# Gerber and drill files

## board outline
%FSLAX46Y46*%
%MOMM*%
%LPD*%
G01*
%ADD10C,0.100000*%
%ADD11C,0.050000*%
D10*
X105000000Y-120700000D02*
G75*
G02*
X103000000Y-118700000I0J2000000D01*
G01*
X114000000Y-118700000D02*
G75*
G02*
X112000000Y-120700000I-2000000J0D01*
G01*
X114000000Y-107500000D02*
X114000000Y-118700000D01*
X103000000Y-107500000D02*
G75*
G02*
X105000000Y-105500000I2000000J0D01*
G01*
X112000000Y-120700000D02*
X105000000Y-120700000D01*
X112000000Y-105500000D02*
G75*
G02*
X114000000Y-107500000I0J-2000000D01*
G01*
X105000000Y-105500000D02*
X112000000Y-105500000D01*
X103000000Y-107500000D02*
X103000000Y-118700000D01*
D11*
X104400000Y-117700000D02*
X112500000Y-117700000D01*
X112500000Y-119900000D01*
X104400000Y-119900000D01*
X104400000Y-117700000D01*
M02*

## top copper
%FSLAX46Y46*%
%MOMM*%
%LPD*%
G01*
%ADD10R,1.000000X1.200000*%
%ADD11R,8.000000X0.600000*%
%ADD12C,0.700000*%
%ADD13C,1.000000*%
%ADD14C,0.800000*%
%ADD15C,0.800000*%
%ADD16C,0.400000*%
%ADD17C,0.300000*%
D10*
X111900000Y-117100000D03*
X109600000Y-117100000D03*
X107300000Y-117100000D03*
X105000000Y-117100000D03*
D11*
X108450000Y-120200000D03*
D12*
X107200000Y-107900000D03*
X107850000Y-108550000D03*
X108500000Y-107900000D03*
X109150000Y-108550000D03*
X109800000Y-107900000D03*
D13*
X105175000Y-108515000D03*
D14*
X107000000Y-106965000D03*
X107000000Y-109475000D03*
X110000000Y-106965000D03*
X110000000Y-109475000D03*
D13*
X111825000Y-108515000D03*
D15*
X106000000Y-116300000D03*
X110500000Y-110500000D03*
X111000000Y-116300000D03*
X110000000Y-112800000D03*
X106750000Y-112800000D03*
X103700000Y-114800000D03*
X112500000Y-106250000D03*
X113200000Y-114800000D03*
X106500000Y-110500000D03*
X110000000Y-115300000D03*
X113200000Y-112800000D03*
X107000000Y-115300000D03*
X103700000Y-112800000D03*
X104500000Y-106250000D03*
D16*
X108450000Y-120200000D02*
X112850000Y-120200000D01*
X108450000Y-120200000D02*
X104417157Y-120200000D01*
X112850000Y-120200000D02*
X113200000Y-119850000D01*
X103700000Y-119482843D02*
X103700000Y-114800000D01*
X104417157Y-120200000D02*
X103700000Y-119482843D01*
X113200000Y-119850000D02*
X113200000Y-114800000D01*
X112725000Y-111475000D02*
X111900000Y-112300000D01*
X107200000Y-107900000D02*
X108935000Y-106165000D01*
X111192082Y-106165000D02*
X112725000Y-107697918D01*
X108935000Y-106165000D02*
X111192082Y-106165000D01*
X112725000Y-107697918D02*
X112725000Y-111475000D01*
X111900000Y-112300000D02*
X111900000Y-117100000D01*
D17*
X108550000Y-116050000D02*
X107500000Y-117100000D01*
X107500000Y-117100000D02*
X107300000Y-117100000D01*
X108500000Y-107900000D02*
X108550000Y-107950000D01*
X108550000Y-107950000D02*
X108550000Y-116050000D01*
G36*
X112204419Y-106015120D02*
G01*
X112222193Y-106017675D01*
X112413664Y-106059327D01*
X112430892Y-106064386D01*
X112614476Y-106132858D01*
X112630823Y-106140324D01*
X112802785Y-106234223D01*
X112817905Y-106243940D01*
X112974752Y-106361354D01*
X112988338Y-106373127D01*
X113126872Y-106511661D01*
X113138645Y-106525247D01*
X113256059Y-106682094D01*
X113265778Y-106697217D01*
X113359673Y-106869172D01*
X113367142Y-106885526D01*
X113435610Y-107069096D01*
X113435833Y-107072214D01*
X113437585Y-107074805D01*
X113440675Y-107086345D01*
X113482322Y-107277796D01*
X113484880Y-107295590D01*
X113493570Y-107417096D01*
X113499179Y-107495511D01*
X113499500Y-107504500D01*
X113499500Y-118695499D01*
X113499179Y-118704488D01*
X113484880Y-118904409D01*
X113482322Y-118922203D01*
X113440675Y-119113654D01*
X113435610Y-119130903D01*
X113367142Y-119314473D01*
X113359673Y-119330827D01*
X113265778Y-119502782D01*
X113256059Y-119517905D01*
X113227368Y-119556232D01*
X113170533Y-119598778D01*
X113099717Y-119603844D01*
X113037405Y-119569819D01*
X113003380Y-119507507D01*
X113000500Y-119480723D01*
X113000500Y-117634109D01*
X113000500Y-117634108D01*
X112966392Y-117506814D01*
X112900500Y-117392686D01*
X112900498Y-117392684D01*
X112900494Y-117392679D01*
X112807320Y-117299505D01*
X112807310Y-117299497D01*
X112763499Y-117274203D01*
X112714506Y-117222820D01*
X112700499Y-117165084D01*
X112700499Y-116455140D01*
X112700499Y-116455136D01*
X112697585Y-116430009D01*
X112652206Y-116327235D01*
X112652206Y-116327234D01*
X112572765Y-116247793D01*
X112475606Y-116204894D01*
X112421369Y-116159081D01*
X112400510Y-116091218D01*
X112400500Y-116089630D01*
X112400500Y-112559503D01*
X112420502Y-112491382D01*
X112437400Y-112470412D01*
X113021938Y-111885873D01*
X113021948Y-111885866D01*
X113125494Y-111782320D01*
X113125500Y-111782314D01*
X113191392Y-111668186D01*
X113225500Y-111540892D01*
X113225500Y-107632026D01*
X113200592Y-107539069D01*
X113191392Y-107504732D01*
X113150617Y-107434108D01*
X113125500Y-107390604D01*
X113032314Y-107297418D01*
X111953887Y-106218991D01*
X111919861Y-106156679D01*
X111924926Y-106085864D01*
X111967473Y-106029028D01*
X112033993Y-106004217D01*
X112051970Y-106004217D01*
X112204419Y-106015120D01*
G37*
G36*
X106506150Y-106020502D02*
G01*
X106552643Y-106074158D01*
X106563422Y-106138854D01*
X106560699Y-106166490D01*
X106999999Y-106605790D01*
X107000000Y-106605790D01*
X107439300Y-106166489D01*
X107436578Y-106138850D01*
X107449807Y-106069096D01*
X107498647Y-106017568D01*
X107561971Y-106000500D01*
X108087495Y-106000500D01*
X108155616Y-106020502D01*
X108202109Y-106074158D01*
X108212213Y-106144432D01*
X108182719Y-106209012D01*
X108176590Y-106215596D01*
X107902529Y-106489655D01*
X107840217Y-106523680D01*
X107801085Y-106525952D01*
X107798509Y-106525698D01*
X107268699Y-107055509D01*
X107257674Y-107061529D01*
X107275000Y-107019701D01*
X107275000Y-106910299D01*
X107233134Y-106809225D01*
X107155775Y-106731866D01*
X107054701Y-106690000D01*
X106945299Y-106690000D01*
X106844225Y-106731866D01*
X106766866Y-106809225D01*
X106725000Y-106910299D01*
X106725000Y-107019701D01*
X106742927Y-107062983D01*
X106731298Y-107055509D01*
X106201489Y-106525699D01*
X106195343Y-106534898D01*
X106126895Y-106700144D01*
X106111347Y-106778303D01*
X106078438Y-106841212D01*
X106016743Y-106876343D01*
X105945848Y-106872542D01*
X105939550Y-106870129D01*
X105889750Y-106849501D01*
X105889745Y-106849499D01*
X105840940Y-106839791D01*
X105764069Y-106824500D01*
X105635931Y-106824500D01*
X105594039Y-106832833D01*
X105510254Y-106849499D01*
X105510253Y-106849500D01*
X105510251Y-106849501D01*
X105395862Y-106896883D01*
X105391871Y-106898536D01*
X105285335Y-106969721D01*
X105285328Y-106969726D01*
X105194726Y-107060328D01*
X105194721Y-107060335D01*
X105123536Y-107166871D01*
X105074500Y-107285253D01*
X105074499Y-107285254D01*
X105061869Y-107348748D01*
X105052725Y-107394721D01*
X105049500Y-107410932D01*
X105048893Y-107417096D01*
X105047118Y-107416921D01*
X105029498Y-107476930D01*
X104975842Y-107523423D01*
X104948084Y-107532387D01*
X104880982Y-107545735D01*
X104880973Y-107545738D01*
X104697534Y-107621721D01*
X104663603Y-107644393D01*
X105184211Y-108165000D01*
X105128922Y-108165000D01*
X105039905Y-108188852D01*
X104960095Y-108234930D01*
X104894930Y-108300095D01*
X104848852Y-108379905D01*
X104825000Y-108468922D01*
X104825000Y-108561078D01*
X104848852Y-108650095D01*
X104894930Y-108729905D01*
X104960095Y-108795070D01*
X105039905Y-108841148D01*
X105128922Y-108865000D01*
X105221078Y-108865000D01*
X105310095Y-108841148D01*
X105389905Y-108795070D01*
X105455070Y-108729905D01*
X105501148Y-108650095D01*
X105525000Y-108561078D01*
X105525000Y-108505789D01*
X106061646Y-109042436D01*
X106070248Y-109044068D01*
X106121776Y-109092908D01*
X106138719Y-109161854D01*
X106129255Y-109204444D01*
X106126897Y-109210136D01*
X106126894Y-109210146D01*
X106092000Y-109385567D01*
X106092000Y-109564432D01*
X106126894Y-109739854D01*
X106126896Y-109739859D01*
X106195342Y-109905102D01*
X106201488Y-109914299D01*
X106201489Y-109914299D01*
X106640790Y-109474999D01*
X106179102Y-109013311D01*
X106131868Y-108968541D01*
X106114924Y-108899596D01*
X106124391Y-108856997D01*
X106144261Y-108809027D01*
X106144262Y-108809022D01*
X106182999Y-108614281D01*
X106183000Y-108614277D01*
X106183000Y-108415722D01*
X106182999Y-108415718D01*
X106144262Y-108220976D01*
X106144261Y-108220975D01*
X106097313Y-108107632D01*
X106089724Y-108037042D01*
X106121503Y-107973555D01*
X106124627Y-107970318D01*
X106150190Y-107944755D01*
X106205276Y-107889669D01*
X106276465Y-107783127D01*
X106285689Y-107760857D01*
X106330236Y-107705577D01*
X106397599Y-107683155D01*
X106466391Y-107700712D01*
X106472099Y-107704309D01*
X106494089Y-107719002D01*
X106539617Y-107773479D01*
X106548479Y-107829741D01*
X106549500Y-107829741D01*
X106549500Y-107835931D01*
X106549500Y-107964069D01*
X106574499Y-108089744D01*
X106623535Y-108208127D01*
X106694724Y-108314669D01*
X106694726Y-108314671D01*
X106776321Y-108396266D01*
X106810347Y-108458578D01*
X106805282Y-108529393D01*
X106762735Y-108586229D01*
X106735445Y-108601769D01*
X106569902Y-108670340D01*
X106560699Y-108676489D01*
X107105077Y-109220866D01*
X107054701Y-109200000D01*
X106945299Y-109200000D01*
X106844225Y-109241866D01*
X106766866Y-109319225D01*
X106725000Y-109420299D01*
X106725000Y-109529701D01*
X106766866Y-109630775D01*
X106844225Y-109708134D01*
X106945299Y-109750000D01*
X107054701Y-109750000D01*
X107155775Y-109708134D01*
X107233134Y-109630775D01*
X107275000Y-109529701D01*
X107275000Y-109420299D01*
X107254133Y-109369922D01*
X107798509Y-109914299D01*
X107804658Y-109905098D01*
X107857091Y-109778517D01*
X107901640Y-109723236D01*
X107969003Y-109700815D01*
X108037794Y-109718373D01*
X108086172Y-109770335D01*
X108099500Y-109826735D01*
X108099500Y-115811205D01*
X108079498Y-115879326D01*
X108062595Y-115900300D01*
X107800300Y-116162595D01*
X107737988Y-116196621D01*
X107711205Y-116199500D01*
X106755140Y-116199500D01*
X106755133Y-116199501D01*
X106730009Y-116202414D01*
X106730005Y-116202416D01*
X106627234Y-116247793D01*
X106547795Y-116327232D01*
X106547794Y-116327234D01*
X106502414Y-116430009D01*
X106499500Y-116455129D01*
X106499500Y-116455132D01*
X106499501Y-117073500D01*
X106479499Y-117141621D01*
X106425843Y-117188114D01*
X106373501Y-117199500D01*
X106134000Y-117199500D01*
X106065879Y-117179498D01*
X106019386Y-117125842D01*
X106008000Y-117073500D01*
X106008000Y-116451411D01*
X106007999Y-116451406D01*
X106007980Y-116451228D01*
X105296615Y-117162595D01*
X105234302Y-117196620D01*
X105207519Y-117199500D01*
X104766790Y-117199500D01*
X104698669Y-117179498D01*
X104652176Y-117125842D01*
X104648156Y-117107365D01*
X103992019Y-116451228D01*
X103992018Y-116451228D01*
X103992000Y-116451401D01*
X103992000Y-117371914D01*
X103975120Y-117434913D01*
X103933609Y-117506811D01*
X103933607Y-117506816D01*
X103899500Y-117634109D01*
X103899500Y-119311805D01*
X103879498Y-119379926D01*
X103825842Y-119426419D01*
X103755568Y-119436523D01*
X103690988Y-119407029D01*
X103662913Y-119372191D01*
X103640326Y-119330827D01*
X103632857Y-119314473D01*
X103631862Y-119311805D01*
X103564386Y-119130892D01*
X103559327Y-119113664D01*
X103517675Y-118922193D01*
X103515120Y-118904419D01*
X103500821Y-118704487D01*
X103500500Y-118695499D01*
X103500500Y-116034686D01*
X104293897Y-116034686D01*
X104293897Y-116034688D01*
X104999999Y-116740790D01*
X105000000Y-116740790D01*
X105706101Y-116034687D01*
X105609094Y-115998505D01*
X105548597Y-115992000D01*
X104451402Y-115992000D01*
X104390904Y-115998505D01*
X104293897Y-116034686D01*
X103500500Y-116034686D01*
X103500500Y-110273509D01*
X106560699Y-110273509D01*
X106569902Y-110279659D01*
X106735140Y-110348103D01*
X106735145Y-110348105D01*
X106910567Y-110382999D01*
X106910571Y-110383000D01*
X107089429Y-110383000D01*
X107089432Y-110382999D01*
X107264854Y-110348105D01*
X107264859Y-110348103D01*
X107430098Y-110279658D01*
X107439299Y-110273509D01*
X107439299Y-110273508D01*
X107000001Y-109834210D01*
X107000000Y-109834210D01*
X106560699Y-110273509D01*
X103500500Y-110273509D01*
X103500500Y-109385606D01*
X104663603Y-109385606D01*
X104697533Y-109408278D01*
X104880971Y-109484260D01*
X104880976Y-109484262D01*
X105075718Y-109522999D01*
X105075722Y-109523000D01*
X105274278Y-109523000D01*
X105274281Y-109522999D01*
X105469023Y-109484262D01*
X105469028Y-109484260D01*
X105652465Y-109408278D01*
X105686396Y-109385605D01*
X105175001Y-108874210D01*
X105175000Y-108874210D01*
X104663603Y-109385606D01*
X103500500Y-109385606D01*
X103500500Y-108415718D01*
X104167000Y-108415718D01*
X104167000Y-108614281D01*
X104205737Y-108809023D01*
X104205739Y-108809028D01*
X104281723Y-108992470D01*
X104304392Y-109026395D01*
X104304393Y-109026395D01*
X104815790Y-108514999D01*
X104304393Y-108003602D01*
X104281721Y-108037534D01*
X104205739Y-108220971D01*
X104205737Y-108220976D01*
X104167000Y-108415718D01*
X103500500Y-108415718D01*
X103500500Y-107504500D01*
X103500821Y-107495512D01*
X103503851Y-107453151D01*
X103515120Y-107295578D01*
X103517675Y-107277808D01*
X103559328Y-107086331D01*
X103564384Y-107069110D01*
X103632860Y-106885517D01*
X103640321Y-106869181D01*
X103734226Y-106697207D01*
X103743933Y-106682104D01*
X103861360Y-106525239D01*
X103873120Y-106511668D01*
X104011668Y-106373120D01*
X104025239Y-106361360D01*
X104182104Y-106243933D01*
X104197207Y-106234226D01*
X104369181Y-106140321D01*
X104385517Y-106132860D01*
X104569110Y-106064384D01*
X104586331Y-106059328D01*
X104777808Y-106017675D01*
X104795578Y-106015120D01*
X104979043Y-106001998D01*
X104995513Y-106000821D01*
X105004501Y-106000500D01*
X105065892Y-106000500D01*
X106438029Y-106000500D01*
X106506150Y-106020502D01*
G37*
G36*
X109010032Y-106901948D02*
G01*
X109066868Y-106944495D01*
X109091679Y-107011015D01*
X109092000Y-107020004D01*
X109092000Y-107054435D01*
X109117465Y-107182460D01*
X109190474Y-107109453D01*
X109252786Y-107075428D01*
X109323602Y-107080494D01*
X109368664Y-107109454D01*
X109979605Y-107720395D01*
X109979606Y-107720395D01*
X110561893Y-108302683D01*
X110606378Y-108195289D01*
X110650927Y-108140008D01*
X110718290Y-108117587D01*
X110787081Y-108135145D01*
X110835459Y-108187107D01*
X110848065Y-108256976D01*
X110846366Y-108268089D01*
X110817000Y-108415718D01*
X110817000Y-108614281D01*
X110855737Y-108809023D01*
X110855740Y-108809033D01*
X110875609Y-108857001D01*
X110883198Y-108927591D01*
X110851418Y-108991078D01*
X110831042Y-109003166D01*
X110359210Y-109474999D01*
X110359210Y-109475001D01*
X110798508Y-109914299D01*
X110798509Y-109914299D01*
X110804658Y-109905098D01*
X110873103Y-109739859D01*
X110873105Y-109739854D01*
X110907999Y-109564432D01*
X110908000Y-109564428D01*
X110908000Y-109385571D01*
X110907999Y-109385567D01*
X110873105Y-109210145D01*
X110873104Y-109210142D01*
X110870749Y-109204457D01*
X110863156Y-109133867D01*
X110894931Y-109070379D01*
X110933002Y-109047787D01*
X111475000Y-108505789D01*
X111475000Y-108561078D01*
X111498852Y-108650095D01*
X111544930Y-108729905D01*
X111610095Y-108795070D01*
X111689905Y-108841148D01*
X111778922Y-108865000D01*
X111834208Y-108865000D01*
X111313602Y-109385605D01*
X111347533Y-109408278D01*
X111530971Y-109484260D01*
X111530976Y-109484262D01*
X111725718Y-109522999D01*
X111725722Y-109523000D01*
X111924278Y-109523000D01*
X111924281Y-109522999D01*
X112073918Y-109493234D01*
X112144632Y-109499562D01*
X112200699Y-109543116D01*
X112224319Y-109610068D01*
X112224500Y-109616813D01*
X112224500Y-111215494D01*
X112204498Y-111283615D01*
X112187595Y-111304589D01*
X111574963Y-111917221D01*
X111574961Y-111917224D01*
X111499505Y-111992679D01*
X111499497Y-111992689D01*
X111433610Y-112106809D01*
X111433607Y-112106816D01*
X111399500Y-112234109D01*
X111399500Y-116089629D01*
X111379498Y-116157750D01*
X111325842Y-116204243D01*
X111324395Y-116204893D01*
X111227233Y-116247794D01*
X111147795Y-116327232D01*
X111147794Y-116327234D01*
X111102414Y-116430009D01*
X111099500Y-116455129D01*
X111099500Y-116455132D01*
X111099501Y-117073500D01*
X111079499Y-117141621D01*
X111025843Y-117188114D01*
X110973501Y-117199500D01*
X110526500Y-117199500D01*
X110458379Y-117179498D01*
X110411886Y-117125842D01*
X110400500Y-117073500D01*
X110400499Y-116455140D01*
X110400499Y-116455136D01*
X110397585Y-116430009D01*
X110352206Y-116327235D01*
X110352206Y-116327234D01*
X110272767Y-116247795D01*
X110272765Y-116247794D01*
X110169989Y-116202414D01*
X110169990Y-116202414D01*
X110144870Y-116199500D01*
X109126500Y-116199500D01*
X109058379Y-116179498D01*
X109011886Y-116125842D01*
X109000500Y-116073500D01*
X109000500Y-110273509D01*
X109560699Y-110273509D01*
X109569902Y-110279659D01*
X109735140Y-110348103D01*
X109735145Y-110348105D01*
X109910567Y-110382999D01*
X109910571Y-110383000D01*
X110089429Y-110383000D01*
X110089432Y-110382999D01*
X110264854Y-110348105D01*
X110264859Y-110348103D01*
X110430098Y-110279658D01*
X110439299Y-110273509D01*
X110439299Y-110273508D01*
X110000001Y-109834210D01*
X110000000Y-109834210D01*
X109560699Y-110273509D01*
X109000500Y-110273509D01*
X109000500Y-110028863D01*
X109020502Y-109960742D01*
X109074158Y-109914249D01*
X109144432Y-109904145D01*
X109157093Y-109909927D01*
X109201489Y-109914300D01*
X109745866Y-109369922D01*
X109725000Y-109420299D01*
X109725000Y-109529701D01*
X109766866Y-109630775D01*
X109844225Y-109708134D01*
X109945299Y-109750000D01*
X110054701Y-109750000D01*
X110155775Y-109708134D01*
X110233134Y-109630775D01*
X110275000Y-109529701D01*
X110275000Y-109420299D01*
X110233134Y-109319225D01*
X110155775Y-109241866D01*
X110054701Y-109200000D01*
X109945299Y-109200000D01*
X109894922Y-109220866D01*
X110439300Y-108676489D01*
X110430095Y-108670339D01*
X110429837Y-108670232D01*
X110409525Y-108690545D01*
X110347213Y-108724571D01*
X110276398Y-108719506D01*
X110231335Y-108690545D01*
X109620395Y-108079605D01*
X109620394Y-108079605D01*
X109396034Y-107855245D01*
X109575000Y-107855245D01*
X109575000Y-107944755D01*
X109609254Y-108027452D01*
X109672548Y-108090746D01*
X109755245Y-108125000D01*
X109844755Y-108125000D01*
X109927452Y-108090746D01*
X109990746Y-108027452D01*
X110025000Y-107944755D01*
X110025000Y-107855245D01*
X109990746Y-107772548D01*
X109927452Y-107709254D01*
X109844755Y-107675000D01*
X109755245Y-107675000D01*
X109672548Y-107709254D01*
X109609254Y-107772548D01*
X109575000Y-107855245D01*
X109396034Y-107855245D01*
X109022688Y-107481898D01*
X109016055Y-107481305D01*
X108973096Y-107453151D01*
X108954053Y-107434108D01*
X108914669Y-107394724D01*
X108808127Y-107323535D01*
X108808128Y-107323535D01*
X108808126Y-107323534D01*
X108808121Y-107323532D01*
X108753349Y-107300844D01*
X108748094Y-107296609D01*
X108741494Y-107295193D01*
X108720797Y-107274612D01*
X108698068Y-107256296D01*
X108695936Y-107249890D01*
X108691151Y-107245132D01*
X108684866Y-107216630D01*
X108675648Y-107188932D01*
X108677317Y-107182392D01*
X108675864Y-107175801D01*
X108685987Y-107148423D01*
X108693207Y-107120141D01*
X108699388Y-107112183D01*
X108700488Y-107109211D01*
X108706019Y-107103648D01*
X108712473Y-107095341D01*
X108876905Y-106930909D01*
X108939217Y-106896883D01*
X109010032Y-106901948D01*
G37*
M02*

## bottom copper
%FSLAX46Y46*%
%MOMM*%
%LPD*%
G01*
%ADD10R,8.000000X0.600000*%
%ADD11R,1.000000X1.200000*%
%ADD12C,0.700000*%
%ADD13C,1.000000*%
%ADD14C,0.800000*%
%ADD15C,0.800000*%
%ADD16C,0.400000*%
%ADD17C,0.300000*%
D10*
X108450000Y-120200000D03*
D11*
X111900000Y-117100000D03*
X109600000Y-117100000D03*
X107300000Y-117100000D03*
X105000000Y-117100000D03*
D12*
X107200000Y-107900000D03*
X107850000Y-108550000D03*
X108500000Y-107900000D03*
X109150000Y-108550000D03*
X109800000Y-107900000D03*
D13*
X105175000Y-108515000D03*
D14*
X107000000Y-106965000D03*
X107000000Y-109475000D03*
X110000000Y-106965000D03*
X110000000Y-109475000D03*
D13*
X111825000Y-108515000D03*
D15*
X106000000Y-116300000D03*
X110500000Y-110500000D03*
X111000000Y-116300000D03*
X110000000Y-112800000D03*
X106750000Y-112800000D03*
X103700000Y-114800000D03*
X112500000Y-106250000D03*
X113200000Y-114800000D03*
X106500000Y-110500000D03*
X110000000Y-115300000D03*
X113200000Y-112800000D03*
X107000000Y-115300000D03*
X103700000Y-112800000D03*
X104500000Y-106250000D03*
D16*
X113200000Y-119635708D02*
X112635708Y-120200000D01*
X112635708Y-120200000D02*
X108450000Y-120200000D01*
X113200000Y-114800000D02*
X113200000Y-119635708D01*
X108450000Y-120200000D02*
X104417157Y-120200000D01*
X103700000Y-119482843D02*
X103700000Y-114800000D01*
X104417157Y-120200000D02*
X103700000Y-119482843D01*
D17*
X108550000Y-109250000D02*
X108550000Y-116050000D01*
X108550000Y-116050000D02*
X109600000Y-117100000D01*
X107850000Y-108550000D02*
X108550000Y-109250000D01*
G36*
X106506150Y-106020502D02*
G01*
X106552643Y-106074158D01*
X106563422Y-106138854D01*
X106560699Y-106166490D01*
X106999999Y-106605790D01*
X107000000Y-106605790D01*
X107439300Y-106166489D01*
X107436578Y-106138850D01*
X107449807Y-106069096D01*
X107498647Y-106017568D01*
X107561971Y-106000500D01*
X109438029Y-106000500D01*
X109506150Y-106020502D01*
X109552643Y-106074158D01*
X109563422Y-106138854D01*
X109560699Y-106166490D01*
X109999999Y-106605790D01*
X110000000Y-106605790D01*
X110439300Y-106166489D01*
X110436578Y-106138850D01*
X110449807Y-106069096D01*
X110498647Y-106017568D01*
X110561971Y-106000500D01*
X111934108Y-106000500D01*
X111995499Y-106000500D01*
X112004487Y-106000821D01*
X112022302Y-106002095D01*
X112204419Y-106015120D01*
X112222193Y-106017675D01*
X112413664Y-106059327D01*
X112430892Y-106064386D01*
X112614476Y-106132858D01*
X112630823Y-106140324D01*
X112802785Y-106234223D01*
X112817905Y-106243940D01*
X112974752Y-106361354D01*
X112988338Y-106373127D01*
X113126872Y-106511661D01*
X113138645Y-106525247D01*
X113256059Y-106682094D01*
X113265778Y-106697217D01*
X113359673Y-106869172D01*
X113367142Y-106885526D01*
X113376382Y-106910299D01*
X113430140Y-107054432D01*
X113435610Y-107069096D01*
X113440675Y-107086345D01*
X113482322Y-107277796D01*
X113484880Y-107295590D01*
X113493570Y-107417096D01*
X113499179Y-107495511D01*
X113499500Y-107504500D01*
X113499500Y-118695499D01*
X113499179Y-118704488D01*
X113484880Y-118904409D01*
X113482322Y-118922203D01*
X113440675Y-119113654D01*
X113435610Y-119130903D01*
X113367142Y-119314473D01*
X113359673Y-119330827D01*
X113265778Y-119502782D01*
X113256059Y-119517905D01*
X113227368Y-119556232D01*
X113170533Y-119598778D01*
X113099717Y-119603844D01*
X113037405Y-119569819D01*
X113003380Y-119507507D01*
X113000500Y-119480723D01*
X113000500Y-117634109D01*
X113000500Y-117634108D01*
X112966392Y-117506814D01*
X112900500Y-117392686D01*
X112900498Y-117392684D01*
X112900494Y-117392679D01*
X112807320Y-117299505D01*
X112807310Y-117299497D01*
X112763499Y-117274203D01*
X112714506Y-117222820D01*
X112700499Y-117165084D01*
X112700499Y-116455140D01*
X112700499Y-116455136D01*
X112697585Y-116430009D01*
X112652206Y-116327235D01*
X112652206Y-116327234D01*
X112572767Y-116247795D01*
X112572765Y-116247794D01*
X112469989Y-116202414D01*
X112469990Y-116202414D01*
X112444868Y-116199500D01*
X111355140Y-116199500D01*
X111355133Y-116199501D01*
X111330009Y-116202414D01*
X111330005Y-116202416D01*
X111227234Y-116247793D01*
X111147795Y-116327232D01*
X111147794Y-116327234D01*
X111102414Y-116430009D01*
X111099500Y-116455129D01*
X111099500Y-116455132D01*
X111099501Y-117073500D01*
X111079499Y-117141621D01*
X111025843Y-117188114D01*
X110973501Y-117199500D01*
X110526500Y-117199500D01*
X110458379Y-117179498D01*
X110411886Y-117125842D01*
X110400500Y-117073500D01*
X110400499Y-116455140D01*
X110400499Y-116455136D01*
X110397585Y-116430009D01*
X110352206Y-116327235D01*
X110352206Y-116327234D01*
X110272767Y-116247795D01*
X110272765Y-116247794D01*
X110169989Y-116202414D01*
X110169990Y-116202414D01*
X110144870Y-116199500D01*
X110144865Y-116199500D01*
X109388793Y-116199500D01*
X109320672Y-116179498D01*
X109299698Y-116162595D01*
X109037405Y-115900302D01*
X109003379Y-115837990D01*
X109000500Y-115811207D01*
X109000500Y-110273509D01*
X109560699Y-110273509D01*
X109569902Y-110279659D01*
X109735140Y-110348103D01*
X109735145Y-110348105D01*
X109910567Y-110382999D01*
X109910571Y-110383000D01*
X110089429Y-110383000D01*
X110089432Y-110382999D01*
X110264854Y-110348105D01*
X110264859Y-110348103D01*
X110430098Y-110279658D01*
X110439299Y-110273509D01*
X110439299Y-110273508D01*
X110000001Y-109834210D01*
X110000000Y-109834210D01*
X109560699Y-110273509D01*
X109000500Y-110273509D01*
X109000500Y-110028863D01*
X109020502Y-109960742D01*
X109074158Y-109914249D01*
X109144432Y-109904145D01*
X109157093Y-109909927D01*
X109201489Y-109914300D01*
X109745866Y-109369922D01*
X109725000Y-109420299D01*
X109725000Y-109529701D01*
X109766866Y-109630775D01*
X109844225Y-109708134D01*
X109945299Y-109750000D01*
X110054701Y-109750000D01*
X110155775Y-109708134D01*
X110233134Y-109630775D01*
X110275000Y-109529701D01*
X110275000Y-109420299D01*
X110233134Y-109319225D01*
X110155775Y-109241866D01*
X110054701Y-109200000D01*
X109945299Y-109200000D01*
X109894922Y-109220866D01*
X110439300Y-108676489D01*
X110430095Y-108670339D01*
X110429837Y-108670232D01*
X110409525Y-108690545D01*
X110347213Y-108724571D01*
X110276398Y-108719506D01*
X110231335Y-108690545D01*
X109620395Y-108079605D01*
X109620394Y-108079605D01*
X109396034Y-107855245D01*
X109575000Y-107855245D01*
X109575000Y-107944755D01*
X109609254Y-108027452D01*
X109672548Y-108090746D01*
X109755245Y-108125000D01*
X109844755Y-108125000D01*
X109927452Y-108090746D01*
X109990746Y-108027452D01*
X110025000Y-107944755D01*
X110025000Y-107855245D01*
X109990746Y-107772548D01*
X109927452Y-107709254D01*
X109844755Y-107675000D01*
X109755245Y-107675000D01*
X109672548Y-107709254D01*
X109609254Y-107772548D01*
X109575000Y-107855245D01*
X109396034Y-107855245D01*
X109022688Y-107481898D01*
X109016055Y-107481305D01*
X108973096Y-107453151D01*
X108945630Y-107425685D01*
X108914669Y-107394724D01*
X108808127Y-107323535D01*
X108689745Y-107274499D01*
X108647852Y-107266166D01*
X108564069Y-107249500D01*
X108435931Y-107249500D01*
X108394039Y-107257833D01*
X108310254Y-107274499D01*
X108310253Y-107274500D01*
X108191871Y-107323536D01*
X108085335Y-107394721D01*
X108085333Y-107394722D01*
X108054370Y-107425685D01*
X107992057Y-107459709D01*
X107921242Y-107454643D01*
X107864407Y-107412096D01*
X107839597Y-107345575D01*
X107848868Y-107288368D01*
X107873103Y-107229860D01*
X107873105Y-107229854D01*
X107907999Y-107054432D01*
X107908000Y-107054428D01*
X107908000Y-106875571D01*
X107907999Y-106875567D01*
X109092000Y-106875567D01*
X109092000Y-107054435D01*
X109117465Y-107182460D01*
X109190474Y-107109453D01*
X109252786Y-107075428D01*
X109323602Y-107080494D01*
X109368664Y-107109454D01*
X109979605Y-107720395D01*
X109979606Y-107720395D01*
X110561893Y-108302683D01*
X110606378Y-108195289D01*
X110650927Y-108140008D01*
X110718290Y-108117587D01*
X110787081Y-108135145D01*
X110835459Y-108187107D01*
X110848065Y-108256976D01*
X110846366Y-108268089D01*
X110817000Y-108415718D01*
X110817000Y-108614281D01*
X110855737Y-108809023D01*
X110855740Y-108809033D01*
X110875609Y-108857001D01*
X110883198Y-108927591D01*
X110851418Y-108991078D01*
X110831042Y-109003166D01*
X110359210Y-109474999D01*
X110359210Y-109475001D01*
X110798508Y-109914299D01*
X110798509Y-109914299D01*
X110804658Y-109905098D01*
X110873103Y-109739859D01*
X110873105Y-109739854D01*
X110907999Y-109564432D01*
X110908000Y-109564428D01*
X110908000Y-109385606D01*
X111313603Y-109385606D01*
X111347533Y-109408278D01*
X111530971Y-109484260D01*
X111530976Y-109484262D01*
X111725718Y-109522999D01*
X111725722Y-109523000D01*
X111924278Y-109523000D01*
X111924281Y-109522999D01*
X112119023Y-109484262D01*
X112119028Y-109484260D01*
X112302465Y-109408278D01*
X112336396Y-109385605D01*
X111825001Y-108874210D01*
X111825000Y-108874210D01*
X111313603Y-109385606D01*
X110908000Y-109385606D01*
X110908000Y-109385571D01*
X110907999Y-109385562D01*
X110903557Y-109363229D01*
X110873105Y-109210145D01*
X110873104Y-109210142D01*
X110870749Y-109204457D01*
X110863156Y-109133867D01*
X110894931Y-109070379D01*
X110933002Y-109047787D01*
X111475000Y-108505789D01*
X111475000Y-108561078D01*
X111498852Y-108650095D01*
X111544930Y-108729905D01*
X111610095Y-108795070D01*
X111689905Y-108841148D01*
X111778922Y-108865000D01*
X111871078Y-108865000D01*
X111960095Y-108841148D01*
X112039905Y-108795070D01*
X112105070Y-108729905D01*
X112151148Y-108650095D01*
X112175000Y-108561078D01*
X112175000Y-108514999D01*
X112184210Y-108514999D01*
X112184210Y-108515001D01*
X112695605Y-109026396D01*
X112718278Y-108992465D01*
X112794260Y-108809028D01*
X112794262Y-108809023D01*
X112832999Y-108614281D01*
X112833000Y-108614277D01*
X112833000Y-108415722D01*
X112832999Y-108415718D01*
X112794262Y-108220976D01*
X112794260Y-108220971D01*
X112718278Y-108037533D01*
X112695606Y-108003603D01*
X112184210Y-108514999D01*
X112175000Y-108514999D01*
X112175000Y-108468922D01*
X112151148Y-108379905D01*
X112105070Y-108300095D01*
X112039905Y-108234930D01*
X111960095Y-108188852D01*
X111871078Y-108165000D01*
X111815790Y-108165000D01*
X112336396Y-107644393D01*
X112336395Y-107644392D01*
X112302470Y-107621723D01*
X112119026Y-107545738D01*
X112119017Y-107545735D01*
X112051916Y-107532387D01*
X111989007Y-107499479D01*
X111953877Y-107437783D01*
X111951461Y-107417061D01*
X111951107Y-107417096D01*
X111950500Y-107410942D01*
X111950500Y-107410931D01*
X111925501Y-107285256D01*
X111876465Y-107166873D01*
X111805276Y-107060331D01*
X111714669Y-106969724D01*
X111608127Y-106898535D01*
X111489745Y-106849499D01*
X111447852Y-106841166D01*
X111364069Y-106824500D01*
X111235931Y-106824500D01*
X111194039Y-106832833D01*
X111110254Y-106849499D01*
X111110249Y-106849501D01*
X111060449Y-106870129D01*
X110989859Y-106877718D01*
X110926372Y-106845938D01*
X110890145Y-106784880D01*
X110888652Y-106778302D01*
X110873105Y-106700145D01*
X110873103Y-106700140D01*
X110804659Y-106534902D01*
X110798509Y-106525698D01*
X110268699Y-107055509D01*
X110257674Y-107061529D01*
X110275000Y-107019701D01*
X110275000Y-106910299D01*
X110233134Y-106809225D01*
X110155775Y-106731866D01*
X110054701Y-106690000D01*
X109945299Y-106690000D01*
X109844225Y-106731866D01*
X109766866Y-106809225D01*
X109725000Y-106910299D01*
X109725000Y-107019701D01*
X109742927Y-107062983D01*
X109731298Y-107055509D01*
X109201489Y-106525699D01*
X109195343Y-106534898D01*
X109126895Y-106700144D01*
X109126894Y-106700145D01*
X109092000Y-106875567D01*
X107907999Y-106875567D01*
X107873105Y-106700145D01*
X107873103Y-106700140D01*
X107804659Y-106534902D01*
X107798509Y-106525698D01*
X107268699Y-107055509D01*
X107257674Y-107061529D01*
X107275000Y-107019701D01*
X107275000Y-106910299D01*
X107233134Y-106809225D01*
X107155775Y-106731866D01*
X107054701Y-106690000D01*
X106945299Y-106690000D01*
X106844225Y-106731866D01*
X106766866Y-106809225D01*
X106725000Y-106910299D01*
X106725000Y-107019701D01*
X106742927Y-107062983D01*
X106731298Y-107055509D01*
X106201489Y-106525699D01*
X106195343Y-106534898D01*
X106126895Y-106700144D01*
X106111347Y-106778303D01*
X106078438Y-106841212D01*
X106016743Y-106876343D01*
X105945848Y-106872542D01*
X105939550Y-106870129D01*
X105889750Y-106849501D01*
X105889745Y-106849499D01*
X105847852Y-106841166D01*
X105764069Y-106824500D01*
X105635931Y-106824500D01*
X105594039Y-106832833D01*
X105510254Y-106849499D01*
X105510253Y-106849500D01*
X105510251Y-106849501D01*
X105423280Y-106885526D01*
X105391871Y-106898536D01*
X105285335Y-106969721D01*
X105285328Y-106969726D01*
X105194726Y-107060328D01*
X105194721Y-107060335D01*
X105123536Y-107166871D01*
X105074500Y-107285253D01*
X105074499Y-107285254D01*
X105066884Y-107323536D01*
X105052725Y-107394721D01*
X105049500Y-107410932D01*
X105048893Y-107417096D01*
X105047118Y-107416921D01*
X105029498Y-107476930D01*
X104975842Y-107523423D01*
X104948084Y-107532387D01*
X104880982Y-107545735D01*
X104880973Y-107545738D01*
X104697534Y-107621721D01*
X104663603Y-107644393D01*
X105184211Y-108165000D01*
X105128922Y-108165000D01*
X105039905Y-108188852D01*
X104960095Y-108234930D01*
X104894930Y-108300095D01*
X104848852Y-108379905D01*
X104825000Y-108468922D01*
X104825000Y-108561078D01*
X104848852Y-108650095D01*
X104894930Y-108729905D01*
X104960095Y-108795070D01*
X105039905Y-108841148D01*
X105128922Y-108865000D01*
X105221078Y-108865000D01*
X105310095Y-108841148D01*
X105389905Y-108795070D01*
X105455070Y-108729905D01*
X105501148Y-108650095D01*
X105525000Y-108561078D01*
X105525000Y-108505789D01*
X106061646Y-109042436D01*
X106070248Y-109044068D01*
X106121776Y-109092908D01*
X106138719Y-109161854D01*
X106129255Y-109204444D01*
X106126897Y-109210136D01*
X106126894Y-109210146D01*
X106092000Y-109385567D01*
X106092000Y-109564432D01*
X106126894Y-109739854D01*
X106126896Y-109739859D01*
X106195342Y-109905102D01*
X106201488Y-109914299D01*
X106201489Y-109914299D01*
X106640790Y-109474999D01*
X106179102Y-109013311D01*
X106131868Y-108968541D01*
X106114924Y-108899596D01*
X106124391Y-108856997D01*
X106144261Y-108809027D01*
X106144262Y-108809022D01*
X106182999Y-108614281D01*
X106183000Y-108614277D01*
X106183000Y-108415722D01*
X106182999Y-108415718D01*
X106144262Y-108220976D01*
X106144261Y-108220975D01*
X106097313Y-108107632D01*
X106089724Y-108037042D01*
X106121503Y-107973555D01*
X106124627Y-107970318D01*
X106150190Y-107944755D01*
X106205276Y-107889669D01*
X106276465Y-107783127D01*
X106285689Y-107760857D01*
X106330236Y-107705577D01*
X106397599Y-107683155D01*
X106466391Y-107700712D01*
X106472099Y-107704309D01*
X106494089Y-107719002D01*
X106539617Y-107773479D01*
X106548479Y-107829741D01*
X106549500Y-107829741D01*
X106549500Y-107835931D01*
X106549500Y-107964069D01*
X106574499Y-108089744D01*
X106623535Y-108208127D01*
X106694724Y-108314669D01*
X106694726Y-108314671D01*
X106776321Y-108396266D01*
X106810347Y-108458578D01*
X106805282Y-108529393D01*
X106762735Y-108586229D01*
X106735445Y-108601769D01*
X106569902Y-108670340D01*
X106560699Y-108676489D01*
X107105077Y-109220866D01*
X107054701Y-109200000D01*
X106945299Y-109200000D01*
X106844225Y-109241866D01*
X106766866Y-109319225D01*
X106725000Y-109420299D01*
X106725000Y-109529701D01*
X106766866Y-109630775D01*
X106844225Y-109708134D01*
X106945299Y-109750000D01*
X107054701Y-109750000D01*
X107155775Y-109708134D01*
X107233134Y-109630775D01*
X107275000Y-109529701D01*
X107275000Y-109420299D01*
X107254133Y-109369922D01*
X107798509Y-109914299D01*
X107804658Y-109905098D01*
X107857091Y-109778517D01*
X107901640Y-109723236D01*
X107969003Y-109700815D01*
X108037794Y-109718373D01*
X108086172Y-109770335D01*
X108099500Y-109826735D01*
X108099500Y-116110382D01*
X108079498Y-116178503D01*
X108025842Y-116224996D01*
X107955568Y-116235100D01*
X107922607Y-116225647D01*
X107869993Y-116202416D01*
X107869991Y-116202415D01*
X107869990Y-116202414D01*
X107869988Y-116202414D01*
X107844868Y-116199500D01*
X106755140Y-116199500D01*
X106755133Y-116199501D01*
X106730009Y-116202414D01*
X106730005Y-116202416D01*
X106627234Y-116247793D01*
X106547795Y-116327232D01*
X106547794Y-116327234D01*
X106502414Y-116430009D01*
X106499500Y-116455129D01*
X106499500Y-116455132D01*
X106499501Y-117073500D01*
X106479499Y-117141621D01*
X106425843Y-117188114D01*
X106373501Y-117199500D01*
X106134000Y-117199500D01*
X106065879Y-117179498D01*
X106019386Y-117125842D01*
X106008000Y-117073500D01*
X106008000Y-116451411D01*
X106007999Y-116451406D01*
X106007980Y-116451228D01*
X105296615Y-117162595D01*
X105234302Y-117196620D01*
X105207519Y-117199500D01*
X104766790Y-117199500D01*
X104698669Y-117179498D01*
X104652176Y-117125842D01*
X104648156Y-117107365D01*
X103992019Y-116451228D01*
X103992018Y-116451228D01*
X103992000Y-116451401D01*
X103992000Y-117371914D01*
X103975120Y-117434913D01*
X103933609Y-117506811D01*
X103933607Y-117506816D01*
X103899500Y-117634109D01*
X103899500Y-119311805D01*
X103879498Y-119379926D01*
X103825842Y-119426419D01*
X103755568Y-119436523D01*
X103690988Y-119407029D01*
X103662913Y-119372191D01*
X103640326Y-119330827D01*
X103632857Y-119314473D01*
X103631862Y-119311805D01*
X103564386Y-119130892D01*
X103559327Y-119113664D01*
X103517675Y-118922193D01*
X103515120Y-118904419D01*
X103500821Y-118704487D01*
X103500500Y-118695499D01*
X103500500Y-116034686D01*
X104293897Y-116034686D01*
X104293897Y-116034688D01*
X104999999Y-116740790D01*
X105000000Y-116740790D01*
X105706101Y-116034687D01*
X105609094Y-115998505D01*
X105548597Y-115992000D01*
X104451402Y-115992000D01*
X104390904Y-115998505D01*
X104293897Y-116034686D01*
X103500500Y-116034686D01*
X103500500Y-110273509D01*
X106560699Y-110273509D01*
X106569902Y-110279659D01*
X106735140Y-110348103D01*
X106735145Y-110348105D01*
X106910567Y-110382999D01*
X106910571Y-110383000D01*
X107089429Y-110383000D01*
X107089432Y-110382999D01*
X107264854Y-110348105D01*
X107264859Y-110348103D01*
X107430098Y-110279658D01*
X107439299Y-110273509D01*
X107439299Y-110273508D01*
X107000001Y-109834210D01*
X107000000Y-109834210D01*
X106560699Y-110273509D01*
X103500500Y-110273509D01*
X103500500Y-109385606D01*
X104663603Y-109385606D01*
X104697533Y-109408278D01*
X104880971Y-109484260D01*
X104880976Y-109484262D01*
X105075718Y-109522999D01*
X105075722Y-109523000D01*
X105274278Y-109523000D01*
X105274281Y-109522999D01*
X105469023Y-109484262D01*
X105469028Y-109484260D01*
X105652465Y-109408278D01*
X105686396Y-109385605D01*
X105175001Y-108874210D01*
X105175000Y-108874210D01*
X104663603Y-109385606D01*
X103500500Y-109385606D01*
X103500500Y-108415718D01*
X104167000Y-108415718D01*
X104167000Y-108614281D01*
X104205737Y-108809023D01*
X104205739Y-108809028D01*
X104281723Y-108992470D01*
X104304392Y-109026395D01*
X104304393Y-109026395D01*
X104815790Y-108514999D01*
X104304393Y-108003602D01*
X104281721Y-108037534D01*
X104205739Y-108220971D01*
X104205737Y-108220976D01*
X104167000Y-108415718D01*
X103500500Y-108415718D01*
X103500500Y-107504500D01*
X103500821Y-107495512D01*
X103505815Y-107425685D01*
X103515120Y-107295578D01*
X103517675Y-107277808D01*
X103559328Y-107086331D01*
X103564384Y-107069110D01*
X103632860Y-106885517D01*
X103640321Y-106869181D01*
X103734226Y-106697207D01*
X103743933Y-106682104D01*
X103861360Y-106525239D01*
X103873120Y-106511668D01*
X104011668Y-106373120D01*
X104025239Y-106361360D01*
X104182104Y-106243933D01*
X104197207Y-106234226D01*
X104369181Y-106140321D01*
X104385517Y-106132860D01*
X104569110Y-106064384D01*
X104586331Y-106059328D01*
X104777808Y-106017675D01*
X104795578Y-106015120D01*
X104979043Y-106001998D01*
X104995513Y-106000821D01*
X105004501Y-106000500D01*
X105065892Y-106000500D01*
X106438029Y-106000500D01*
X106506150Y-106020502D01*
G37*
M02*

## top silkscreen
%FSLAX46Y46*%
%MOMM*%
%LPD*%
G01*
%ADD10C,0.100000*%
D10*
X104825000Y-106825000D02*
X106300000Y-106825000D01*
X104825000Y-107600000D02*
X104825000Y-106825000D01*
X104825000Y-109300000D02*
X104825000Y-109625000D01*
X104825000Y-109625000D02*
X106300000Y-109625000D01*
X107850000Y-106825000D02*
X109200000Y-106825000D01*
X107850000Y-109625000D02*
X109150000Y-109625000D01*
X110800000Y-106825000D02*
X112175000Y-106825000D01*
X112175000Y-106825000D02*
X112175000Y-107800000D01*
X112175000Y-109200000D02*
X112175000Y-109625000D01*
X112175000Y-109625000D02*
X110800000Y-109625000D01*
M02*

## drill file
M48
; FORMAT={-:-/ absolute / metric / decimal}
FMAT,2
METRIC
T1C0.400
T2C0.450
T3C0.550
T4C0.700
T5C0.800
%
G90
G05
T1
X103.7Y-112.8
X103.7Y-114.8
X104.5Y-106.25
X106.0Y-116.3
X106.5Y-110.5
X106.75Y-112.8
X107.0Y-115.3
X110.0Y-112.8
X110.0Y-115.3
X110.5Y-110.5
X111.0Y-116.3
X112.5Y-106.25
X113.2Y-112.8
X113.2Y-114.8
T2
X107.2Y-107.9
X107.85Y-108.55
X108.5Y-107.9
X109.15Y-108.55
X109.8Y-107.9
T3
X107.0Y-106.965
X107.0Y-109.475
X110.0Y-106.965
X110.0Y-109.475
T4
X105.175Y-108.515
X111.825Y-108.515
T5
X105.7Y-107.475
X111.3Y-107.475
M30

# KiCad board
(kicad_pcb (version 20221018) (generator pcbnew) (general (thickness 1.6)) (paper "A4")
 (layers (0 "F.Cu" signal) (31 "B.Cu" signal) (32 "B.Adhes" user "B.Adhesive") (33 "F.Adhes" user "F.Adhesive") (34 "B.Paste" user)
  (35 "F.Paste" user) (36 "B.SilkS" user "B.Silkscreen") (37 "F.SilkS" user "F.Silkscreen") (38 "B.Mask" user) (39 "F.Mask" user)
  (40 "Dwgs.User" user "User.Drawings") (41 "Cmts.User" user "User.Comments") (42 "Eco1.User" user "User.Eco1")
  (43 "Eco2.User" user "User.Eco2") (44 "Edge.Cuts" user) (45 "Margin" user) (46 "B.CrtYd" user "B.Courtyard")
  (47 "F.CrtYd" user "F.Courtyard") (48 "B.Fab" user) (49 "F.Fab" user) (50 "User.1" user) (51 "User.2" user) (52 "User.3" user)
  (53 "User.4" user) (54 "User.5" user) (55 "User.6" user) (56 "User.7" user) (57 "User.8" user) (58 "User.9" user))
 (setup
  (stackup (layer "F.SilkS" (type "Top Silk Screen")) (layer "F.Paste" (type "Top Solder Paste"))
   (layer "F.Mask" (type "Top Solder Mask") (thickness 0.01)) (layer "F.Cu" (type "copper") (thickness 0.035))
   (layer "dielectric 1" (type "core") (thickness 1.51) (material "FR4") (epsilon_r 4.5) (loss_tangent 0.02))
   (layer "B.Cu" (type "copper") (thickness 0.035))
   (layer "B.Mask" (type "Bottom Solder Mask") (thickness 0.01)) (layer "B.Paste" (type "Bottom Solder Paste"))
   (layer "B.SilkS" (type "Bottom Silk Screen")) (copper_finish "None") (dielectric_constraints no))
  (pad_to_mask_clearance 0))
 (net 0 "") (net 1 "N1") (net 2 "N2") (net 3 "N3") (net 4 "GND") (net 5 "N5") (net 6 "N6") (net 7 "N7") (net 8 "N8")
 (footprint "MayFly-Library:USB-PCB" (layer "F.Cu") (at 108.5 112.7)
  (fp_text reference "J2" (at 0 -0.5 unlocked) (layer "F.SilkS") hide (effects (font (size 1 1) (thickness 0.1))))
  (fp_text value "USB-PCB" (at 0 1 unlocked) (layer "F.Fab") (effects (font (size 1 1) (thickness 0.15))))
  (fp_rect (start 4 5) (end -4.1 7.2) (stroke (width 0.05) (type default)) (fill none) (layer "Edge.Cuts"))
  (pad "1" smd rect (at 3.4 4.4) (size 1 1.2) (layers "F.Cu" "F.Paste" "F.Mask") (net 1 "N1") (thermal_bridge_angle 45))
  (pad "2" smd rect (at 1.1 4.4) (size 1 1.2) (layers "F.Cu" "F.Paste" "F.Mask") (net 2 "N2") (thermal_bridge_angle 45))
  (pad "3" smd rect (at -1.2 4.4) (size 1 1.2) (layers "F.Cu" "F.Paste" "F.Mask") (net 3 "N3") (thermal_bridge_angle 45))
  (pad "4" smd rect (at -3.5 4.4) (size 1 1.2) (layers "F.Cu" "F.Paste" "F.Mask") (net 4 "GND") (thermal_bridge_angle 45))
  (pad "5" smd rect (at -0.05 7.5) (size 8 0.6) (layers "F.Cu" "F.Paste" "F.Mask") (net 4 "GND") (thermal_bridge_angle 45))
  (pad "6" smd rect (at -0.05 7.5) (size 8 0.6) (layers "B.Cu" "B.Paste" "B.Mask") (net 4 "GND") (thermal_bridge_angle 45))
  (pad "7" smd rect (at 3.4 4.4) (size 1 1.2) (layers "B.Cu" "B.Paste" "B.Mask") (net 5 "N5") (thermal_bridge_angle 45))
  (pad "8" smd rect (at 1.1 4.4) (size 1 1.2) (layers "B.Cu" "B.Paste" "B.Mask") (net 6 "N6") (thermal_bridge_angle 45))
  (pad "9" smd rect (at -1.2 4.4) (size 1 1.2) (layers "B.Cu" "B.Paste" "B.Mask") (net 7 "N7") (thermal_bridge_angle 45))
  (pad "10" smd rect (at -3.5 4.4) (size 1 1.2) (layers "B.Cu" "B.Paste" "B.Mask") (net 4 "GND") (thermal_bridge_angle 45)))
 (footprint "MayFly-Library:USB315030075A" (layer "F.Cu") (at 108.5 107.9)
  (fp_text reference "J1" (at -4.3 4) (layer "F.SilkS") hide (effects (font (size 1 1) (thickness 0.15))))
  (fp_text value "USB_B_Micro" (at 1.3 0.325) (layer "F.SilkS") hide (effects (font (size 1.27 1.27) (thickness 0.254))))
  (fp_line (start -3.675 -1.075) (end -2.2 -1.075) (stroke (width 0.1) (type solid)) (layer "F.SilkS"))
  (fp_line (start -3.675 -0.3) (end -3.675 -1.075) (stroke (width 0.1) (type solid)) (layer "F.SilkS"))
  (fp_line (start -3.675 1.4) (end -3.675 1.725) (stroke (width 0.1) (type solid)) (layer "F.SilkS"))
  (fp_line (start -3.675 1.725) (end -2.2 1.725) (stroke (width 0.1) (type solid)) (layer "F.SilkS"))
  (fp_line (start -0.65 -1.075) (end 0.7 -1.075) (stroke (width 0.1) (type solid)) (layer "F.SilkS"))
  (fp_line (start -0.65 1.725) (end 0.65 1.725) (stroke (width 0.1) (type solid)) (layer "F.SilkS"))
  (fp_line (start 2.3 -1.075) (end 3.675 -1.075) (stroke (width 0.1) (type solid)) (layer "F.SilkS"))
  (fp_line (start 3.675 -1.075) (end 3.675 -0.1) (stroke (width 0.1) (type solid)) (layer "F.SilkS"))
  (fp_line (start 3.675 1.3) (end 3.675 1.725) (stroke (width 0.1) (type solid)) (layer "F.SilkS"))
  (fp_line (start 3.675 1.725) (end 2.3 1.725) (stroke (width 0.1) (type solid)) (layer "F.SilkS"))
  (pad "" np_thru_hole circle (at -2.8 -0.425) (size 0.8 0.8) (drill 0.8) (layers "*.Cu" "*.Mask"))
  (pad "" np_thru_hole circle (at 2.8 -0.425) (size 0.8 0.8) (drill 0.8) (layers "*.Cu" "*.Mask"))
  (pad "1" thru_hole circle (at -1.3 0) (size 0.7 0.7) (drill 0.45) (layers "*.Cu" "*.Mask") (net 1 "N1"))
  (pad "2" thru_hole circle (at -0.65 0.65) (size 0.7 0.7) (drill 0.45) (layers "*.Cu" "*.Mask") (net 6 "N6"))
  (pad "3" thru_hole circle (at 0 0) (size 0.7 0.7) (drill 0.45) (layers "*.Cu" "*.Mask") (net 3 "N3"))
  (pad "4" thru_hole circle (at 0.65 0.65) (size 0.7 0.7) (drill 0.45) (layers "*.Cu" "*.Mask") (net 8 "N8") (clearance 0.05))
  (pad "5" thru_hole circle (at 1.3 0) (size 0.7 0.7) (drill 0.45) (layers "*.Cu" "*.Mask") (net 4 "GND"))
  (pad "6" thru_hole circle (at -3.325 0.615) (size 1 1) (drill 0.7) (layers "*.Cu" "*.Mask") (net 4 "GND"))
  (pad "6" thru_hole circle (at -1.5 -0.935) (size 0.8 0.8) (drill 0.55) (layers "*.Cu" "*.Mask") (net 4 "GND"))
  (pad "6" thru_hole circle (at -1.5 1.575) (size 0.8 0.8) (drill 0.55) (layers "*.Cu" "*.Mask") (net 4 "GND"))
  (pad "6" thru_hole circle (at 1.5 -0.935) (size 0.8 0.8) (drill 0.55) (layers "*.Cu" "*.Mask") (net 4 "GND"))
  (pad "6" thru_hole circle (at 1.5 1.575) (size 0.8 0.8) (drill 0.55) (layers "*.Cu" "*.Mask") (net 4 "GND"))
  (pad "6" thru_hole circle (at 3.325 0.615) (size 1 1) (drill 0.7) (layers "*.Cu" "*.Mask") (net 4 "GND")))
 (gr_arc (start 105 120.7) (mid 103.585786 120.114214) (end 103 118.7) (stroke (width 0.1) (type solid)) (layer "Edge.Cuts"))
 (gr_arc (start 114 118.7) (mid 113.414214 120.114214) (end 112 120.7) (stroke (width 0.1) (type solid)) (layer "Edge.Cuts"))
 (gr_line (start 114 107.5) (end 114 118.7) (stroke (width 0.1) (type default)) (layer "Edge.Cuts"))
 (gr_arc (start 103 107.5) (mid 103.585786 106.085786) (end 105 105.5) (stroke (width 0.1) (type solid)) (layer "Edge.Cuts"))
 (gr_line (start 112 120.7) (end 105 120.7) (stroke (width 0.1) (type default)) (layer "Edge.Cuts"))
 (gr_arc (start 112 105.5) (mid 113.414214 106.085786) (end 114 107.5) (stroke (width 0.1) (type solid)) (layer "Edge.Cuts"))
 (gr_line (start 105 105.5) (end 112 105.5) (stroke (width 0.1) (type default)) (layer "Edge.Cuts"))
 (gr_line (start 103 107.5) (end 103 118.7) (stroke (width 0.1) (type default)) (layer "Edge.Cuts"))
 (segment (start 108.45 120.2) (end 112.85 120.2) (width 0.4) (layer "F.Cu") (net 4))
 (segment (start 108.45 120.2) (end 104.417157 120.2) (width 0.4) (layer "F.Cu") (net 4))
 (segment (start 112.85 120.2) (end 113.2 119.85) (width 0.4) (layer "F.Cu") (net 4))
 (segment (start 103.7 119.482843) (end 103.7 114.8) (width 0.4) (layer "F.Cu") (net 4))
 (segment (start 104.417157 120.2) (end 103.7 119.482843) (width 0.4) (layer "F.Cu") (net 4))
 (segment (start 113.2 119.85) (end 113.2 114.8) (width 0.4) (layer "F.Cu") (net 4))
 (via (at 106 116.3) (size 0.8) (drill 0.4) (layers "F.Cu" "B.Cu") (free) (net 4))
 (via (at 110.5 110.5) (size 0.8) (drill 0.4) (layers "F.Cu" "B.Cu") (free) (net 4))
 (via (at 111 116.3) (size 0.8) (drill 0.4) (layers "F.Cu" "B.Cu") (free) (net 4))
 (via (at 110 112.8) (size 0.8) (drill 0.4) (layers "F.Cu" "B.Cu") (free) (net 4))
 (via (at 106.75 112.8) (size 0.8) (drill 0.4) (layers "F.Cu" "B.Cu") (free) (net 4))
 (via (at 103.7 114.8) (size 0.8) (drill 0.4) (layers "F.Cu" "B.Cu") (free) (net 4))
 (via (at 112.5 106.25) (size 0.8) (drill 0.4) (layers "F.Cu" "B.Cu") (free) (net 4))
 (via (at 113.2 114.8) (size 0.8) (drill 0.4) (layers "F.Cu" "B.Cu") (free) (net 4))
 (via (at 106.5 110.5) (size 0.8) (drill 0.4) (layers "F.Cu" "B.Cu") (free) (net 4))
 (via (at 110 115.3) (size 0.8) (drill 0.4) (layers "F.Cu" "B.Cu") (free) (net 4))
 (via (at 113.2 112.8) (size 0.8) (drill 0.4) (layers "F.Cu" "B.Cu") (free) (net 4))
 (via (at 107 115.3) (size 0.8) (drill 0.4) (layers "F.Cu" "B.Cu") (free) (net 4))
 (via (at 103.7 112.8) (size 0.8) (drill 0.4) (layers "F.Cu" "B.Cu") (free) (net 4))
 (via (at 104.5 106.25) (size 0.8) (drill 0.4) (layers "F.Cu" "B.Cu") (free) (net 4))
 (segment (start 113.2 119.635708) (end 112.635708 120.2) (width 0.4) (layer "B.Cu") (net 4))
 (segment (start 112.635708 120.2) (end 108.45 120.2) (width 0.4) (layer "B.Cu") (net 4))
 (segment (start 113.2 114.8) (end 113.2 119.635708) (width 0.4) (layer "B.Cu") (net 4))
 (segment (start 108.45 120.2) (end 104.417157 120.2) (width 0.4) (layer "B.Cu") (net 4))
 (segment (start 103.7 119.482843) (end 103.7 114.8) (width 0.4) (layer "B.Cu") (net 4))
 (segment (start 104.417157 120.2) (end 103.7 119.482843) (width 0.4) (layer "B.Cu") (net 4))
 (segment (start 112.725 111.475) (end 111.9 112.3) (width 0.4) (layer "F.Cu") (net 1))
 (segment (start 107.2 107.9) (end 108.935 106.165) (width 0.4) (layer "F.Cu") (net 1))
 (segment (start 111.192082 106.165) (end 112.725 107.697918) (width 0.4) (layer "F.Cu") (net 1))
 (segment (start 108.935 106.165) (end 111.192082 106.165) (width 0.4) (layer "F.Cu") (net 1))
 (segment (start 112.725 107.697918) (end 112.725 111.475) (width 0.4) (layer "F.Cu") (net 1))
 (segment (start 111.9 112.3) (end 111.9 117.1) (width 0.4) (layer "F.Cu") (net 1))
 (segment (start 108.55 109.25) (end 108.55 116.05) (width 0.3) (layer "B.Cu") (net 6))
 (segment (start 108.55 116.05) (end 109.6 117.1) (width 0.3) (layer "B.Cu") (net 6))
 (segment (start 107.85 108.55) (end 108.55 109.25) (width 0.3) (layer "B.Cu") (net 6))
 (segment (start 108.55 116.05) (end 107.5 117.1) (width 0.3) (layer "F.Cu") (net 3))
 (segment (start 107.5 117.1) (end 107.3 117.1) (width 0.3) (layer "F.Cu") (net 3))
 (segment (start 108.5 107.9) (end 108.55 107.95) (width 0.3) (layer "F.Cu") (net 3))
 (segment (start 108.55 107.95) (end 108.55 116.05) (width 0.3) (layer "F.Cu") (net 3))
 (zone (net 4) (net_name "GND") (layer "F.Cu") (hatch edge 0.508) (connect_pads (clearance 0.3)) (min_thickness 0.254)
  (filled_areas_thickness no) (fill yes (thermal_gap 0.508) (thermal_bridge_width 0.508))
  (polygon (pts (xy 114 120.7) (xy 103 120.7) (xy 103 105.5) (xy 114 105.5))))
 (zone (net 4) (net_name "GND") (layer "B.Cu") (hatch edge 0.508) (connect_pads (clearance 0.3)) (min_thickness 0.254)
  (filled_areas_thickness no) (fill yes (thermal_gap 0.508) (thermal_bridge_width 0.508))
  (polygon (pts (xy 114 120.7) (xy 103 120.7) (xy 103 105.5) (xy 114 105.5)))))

